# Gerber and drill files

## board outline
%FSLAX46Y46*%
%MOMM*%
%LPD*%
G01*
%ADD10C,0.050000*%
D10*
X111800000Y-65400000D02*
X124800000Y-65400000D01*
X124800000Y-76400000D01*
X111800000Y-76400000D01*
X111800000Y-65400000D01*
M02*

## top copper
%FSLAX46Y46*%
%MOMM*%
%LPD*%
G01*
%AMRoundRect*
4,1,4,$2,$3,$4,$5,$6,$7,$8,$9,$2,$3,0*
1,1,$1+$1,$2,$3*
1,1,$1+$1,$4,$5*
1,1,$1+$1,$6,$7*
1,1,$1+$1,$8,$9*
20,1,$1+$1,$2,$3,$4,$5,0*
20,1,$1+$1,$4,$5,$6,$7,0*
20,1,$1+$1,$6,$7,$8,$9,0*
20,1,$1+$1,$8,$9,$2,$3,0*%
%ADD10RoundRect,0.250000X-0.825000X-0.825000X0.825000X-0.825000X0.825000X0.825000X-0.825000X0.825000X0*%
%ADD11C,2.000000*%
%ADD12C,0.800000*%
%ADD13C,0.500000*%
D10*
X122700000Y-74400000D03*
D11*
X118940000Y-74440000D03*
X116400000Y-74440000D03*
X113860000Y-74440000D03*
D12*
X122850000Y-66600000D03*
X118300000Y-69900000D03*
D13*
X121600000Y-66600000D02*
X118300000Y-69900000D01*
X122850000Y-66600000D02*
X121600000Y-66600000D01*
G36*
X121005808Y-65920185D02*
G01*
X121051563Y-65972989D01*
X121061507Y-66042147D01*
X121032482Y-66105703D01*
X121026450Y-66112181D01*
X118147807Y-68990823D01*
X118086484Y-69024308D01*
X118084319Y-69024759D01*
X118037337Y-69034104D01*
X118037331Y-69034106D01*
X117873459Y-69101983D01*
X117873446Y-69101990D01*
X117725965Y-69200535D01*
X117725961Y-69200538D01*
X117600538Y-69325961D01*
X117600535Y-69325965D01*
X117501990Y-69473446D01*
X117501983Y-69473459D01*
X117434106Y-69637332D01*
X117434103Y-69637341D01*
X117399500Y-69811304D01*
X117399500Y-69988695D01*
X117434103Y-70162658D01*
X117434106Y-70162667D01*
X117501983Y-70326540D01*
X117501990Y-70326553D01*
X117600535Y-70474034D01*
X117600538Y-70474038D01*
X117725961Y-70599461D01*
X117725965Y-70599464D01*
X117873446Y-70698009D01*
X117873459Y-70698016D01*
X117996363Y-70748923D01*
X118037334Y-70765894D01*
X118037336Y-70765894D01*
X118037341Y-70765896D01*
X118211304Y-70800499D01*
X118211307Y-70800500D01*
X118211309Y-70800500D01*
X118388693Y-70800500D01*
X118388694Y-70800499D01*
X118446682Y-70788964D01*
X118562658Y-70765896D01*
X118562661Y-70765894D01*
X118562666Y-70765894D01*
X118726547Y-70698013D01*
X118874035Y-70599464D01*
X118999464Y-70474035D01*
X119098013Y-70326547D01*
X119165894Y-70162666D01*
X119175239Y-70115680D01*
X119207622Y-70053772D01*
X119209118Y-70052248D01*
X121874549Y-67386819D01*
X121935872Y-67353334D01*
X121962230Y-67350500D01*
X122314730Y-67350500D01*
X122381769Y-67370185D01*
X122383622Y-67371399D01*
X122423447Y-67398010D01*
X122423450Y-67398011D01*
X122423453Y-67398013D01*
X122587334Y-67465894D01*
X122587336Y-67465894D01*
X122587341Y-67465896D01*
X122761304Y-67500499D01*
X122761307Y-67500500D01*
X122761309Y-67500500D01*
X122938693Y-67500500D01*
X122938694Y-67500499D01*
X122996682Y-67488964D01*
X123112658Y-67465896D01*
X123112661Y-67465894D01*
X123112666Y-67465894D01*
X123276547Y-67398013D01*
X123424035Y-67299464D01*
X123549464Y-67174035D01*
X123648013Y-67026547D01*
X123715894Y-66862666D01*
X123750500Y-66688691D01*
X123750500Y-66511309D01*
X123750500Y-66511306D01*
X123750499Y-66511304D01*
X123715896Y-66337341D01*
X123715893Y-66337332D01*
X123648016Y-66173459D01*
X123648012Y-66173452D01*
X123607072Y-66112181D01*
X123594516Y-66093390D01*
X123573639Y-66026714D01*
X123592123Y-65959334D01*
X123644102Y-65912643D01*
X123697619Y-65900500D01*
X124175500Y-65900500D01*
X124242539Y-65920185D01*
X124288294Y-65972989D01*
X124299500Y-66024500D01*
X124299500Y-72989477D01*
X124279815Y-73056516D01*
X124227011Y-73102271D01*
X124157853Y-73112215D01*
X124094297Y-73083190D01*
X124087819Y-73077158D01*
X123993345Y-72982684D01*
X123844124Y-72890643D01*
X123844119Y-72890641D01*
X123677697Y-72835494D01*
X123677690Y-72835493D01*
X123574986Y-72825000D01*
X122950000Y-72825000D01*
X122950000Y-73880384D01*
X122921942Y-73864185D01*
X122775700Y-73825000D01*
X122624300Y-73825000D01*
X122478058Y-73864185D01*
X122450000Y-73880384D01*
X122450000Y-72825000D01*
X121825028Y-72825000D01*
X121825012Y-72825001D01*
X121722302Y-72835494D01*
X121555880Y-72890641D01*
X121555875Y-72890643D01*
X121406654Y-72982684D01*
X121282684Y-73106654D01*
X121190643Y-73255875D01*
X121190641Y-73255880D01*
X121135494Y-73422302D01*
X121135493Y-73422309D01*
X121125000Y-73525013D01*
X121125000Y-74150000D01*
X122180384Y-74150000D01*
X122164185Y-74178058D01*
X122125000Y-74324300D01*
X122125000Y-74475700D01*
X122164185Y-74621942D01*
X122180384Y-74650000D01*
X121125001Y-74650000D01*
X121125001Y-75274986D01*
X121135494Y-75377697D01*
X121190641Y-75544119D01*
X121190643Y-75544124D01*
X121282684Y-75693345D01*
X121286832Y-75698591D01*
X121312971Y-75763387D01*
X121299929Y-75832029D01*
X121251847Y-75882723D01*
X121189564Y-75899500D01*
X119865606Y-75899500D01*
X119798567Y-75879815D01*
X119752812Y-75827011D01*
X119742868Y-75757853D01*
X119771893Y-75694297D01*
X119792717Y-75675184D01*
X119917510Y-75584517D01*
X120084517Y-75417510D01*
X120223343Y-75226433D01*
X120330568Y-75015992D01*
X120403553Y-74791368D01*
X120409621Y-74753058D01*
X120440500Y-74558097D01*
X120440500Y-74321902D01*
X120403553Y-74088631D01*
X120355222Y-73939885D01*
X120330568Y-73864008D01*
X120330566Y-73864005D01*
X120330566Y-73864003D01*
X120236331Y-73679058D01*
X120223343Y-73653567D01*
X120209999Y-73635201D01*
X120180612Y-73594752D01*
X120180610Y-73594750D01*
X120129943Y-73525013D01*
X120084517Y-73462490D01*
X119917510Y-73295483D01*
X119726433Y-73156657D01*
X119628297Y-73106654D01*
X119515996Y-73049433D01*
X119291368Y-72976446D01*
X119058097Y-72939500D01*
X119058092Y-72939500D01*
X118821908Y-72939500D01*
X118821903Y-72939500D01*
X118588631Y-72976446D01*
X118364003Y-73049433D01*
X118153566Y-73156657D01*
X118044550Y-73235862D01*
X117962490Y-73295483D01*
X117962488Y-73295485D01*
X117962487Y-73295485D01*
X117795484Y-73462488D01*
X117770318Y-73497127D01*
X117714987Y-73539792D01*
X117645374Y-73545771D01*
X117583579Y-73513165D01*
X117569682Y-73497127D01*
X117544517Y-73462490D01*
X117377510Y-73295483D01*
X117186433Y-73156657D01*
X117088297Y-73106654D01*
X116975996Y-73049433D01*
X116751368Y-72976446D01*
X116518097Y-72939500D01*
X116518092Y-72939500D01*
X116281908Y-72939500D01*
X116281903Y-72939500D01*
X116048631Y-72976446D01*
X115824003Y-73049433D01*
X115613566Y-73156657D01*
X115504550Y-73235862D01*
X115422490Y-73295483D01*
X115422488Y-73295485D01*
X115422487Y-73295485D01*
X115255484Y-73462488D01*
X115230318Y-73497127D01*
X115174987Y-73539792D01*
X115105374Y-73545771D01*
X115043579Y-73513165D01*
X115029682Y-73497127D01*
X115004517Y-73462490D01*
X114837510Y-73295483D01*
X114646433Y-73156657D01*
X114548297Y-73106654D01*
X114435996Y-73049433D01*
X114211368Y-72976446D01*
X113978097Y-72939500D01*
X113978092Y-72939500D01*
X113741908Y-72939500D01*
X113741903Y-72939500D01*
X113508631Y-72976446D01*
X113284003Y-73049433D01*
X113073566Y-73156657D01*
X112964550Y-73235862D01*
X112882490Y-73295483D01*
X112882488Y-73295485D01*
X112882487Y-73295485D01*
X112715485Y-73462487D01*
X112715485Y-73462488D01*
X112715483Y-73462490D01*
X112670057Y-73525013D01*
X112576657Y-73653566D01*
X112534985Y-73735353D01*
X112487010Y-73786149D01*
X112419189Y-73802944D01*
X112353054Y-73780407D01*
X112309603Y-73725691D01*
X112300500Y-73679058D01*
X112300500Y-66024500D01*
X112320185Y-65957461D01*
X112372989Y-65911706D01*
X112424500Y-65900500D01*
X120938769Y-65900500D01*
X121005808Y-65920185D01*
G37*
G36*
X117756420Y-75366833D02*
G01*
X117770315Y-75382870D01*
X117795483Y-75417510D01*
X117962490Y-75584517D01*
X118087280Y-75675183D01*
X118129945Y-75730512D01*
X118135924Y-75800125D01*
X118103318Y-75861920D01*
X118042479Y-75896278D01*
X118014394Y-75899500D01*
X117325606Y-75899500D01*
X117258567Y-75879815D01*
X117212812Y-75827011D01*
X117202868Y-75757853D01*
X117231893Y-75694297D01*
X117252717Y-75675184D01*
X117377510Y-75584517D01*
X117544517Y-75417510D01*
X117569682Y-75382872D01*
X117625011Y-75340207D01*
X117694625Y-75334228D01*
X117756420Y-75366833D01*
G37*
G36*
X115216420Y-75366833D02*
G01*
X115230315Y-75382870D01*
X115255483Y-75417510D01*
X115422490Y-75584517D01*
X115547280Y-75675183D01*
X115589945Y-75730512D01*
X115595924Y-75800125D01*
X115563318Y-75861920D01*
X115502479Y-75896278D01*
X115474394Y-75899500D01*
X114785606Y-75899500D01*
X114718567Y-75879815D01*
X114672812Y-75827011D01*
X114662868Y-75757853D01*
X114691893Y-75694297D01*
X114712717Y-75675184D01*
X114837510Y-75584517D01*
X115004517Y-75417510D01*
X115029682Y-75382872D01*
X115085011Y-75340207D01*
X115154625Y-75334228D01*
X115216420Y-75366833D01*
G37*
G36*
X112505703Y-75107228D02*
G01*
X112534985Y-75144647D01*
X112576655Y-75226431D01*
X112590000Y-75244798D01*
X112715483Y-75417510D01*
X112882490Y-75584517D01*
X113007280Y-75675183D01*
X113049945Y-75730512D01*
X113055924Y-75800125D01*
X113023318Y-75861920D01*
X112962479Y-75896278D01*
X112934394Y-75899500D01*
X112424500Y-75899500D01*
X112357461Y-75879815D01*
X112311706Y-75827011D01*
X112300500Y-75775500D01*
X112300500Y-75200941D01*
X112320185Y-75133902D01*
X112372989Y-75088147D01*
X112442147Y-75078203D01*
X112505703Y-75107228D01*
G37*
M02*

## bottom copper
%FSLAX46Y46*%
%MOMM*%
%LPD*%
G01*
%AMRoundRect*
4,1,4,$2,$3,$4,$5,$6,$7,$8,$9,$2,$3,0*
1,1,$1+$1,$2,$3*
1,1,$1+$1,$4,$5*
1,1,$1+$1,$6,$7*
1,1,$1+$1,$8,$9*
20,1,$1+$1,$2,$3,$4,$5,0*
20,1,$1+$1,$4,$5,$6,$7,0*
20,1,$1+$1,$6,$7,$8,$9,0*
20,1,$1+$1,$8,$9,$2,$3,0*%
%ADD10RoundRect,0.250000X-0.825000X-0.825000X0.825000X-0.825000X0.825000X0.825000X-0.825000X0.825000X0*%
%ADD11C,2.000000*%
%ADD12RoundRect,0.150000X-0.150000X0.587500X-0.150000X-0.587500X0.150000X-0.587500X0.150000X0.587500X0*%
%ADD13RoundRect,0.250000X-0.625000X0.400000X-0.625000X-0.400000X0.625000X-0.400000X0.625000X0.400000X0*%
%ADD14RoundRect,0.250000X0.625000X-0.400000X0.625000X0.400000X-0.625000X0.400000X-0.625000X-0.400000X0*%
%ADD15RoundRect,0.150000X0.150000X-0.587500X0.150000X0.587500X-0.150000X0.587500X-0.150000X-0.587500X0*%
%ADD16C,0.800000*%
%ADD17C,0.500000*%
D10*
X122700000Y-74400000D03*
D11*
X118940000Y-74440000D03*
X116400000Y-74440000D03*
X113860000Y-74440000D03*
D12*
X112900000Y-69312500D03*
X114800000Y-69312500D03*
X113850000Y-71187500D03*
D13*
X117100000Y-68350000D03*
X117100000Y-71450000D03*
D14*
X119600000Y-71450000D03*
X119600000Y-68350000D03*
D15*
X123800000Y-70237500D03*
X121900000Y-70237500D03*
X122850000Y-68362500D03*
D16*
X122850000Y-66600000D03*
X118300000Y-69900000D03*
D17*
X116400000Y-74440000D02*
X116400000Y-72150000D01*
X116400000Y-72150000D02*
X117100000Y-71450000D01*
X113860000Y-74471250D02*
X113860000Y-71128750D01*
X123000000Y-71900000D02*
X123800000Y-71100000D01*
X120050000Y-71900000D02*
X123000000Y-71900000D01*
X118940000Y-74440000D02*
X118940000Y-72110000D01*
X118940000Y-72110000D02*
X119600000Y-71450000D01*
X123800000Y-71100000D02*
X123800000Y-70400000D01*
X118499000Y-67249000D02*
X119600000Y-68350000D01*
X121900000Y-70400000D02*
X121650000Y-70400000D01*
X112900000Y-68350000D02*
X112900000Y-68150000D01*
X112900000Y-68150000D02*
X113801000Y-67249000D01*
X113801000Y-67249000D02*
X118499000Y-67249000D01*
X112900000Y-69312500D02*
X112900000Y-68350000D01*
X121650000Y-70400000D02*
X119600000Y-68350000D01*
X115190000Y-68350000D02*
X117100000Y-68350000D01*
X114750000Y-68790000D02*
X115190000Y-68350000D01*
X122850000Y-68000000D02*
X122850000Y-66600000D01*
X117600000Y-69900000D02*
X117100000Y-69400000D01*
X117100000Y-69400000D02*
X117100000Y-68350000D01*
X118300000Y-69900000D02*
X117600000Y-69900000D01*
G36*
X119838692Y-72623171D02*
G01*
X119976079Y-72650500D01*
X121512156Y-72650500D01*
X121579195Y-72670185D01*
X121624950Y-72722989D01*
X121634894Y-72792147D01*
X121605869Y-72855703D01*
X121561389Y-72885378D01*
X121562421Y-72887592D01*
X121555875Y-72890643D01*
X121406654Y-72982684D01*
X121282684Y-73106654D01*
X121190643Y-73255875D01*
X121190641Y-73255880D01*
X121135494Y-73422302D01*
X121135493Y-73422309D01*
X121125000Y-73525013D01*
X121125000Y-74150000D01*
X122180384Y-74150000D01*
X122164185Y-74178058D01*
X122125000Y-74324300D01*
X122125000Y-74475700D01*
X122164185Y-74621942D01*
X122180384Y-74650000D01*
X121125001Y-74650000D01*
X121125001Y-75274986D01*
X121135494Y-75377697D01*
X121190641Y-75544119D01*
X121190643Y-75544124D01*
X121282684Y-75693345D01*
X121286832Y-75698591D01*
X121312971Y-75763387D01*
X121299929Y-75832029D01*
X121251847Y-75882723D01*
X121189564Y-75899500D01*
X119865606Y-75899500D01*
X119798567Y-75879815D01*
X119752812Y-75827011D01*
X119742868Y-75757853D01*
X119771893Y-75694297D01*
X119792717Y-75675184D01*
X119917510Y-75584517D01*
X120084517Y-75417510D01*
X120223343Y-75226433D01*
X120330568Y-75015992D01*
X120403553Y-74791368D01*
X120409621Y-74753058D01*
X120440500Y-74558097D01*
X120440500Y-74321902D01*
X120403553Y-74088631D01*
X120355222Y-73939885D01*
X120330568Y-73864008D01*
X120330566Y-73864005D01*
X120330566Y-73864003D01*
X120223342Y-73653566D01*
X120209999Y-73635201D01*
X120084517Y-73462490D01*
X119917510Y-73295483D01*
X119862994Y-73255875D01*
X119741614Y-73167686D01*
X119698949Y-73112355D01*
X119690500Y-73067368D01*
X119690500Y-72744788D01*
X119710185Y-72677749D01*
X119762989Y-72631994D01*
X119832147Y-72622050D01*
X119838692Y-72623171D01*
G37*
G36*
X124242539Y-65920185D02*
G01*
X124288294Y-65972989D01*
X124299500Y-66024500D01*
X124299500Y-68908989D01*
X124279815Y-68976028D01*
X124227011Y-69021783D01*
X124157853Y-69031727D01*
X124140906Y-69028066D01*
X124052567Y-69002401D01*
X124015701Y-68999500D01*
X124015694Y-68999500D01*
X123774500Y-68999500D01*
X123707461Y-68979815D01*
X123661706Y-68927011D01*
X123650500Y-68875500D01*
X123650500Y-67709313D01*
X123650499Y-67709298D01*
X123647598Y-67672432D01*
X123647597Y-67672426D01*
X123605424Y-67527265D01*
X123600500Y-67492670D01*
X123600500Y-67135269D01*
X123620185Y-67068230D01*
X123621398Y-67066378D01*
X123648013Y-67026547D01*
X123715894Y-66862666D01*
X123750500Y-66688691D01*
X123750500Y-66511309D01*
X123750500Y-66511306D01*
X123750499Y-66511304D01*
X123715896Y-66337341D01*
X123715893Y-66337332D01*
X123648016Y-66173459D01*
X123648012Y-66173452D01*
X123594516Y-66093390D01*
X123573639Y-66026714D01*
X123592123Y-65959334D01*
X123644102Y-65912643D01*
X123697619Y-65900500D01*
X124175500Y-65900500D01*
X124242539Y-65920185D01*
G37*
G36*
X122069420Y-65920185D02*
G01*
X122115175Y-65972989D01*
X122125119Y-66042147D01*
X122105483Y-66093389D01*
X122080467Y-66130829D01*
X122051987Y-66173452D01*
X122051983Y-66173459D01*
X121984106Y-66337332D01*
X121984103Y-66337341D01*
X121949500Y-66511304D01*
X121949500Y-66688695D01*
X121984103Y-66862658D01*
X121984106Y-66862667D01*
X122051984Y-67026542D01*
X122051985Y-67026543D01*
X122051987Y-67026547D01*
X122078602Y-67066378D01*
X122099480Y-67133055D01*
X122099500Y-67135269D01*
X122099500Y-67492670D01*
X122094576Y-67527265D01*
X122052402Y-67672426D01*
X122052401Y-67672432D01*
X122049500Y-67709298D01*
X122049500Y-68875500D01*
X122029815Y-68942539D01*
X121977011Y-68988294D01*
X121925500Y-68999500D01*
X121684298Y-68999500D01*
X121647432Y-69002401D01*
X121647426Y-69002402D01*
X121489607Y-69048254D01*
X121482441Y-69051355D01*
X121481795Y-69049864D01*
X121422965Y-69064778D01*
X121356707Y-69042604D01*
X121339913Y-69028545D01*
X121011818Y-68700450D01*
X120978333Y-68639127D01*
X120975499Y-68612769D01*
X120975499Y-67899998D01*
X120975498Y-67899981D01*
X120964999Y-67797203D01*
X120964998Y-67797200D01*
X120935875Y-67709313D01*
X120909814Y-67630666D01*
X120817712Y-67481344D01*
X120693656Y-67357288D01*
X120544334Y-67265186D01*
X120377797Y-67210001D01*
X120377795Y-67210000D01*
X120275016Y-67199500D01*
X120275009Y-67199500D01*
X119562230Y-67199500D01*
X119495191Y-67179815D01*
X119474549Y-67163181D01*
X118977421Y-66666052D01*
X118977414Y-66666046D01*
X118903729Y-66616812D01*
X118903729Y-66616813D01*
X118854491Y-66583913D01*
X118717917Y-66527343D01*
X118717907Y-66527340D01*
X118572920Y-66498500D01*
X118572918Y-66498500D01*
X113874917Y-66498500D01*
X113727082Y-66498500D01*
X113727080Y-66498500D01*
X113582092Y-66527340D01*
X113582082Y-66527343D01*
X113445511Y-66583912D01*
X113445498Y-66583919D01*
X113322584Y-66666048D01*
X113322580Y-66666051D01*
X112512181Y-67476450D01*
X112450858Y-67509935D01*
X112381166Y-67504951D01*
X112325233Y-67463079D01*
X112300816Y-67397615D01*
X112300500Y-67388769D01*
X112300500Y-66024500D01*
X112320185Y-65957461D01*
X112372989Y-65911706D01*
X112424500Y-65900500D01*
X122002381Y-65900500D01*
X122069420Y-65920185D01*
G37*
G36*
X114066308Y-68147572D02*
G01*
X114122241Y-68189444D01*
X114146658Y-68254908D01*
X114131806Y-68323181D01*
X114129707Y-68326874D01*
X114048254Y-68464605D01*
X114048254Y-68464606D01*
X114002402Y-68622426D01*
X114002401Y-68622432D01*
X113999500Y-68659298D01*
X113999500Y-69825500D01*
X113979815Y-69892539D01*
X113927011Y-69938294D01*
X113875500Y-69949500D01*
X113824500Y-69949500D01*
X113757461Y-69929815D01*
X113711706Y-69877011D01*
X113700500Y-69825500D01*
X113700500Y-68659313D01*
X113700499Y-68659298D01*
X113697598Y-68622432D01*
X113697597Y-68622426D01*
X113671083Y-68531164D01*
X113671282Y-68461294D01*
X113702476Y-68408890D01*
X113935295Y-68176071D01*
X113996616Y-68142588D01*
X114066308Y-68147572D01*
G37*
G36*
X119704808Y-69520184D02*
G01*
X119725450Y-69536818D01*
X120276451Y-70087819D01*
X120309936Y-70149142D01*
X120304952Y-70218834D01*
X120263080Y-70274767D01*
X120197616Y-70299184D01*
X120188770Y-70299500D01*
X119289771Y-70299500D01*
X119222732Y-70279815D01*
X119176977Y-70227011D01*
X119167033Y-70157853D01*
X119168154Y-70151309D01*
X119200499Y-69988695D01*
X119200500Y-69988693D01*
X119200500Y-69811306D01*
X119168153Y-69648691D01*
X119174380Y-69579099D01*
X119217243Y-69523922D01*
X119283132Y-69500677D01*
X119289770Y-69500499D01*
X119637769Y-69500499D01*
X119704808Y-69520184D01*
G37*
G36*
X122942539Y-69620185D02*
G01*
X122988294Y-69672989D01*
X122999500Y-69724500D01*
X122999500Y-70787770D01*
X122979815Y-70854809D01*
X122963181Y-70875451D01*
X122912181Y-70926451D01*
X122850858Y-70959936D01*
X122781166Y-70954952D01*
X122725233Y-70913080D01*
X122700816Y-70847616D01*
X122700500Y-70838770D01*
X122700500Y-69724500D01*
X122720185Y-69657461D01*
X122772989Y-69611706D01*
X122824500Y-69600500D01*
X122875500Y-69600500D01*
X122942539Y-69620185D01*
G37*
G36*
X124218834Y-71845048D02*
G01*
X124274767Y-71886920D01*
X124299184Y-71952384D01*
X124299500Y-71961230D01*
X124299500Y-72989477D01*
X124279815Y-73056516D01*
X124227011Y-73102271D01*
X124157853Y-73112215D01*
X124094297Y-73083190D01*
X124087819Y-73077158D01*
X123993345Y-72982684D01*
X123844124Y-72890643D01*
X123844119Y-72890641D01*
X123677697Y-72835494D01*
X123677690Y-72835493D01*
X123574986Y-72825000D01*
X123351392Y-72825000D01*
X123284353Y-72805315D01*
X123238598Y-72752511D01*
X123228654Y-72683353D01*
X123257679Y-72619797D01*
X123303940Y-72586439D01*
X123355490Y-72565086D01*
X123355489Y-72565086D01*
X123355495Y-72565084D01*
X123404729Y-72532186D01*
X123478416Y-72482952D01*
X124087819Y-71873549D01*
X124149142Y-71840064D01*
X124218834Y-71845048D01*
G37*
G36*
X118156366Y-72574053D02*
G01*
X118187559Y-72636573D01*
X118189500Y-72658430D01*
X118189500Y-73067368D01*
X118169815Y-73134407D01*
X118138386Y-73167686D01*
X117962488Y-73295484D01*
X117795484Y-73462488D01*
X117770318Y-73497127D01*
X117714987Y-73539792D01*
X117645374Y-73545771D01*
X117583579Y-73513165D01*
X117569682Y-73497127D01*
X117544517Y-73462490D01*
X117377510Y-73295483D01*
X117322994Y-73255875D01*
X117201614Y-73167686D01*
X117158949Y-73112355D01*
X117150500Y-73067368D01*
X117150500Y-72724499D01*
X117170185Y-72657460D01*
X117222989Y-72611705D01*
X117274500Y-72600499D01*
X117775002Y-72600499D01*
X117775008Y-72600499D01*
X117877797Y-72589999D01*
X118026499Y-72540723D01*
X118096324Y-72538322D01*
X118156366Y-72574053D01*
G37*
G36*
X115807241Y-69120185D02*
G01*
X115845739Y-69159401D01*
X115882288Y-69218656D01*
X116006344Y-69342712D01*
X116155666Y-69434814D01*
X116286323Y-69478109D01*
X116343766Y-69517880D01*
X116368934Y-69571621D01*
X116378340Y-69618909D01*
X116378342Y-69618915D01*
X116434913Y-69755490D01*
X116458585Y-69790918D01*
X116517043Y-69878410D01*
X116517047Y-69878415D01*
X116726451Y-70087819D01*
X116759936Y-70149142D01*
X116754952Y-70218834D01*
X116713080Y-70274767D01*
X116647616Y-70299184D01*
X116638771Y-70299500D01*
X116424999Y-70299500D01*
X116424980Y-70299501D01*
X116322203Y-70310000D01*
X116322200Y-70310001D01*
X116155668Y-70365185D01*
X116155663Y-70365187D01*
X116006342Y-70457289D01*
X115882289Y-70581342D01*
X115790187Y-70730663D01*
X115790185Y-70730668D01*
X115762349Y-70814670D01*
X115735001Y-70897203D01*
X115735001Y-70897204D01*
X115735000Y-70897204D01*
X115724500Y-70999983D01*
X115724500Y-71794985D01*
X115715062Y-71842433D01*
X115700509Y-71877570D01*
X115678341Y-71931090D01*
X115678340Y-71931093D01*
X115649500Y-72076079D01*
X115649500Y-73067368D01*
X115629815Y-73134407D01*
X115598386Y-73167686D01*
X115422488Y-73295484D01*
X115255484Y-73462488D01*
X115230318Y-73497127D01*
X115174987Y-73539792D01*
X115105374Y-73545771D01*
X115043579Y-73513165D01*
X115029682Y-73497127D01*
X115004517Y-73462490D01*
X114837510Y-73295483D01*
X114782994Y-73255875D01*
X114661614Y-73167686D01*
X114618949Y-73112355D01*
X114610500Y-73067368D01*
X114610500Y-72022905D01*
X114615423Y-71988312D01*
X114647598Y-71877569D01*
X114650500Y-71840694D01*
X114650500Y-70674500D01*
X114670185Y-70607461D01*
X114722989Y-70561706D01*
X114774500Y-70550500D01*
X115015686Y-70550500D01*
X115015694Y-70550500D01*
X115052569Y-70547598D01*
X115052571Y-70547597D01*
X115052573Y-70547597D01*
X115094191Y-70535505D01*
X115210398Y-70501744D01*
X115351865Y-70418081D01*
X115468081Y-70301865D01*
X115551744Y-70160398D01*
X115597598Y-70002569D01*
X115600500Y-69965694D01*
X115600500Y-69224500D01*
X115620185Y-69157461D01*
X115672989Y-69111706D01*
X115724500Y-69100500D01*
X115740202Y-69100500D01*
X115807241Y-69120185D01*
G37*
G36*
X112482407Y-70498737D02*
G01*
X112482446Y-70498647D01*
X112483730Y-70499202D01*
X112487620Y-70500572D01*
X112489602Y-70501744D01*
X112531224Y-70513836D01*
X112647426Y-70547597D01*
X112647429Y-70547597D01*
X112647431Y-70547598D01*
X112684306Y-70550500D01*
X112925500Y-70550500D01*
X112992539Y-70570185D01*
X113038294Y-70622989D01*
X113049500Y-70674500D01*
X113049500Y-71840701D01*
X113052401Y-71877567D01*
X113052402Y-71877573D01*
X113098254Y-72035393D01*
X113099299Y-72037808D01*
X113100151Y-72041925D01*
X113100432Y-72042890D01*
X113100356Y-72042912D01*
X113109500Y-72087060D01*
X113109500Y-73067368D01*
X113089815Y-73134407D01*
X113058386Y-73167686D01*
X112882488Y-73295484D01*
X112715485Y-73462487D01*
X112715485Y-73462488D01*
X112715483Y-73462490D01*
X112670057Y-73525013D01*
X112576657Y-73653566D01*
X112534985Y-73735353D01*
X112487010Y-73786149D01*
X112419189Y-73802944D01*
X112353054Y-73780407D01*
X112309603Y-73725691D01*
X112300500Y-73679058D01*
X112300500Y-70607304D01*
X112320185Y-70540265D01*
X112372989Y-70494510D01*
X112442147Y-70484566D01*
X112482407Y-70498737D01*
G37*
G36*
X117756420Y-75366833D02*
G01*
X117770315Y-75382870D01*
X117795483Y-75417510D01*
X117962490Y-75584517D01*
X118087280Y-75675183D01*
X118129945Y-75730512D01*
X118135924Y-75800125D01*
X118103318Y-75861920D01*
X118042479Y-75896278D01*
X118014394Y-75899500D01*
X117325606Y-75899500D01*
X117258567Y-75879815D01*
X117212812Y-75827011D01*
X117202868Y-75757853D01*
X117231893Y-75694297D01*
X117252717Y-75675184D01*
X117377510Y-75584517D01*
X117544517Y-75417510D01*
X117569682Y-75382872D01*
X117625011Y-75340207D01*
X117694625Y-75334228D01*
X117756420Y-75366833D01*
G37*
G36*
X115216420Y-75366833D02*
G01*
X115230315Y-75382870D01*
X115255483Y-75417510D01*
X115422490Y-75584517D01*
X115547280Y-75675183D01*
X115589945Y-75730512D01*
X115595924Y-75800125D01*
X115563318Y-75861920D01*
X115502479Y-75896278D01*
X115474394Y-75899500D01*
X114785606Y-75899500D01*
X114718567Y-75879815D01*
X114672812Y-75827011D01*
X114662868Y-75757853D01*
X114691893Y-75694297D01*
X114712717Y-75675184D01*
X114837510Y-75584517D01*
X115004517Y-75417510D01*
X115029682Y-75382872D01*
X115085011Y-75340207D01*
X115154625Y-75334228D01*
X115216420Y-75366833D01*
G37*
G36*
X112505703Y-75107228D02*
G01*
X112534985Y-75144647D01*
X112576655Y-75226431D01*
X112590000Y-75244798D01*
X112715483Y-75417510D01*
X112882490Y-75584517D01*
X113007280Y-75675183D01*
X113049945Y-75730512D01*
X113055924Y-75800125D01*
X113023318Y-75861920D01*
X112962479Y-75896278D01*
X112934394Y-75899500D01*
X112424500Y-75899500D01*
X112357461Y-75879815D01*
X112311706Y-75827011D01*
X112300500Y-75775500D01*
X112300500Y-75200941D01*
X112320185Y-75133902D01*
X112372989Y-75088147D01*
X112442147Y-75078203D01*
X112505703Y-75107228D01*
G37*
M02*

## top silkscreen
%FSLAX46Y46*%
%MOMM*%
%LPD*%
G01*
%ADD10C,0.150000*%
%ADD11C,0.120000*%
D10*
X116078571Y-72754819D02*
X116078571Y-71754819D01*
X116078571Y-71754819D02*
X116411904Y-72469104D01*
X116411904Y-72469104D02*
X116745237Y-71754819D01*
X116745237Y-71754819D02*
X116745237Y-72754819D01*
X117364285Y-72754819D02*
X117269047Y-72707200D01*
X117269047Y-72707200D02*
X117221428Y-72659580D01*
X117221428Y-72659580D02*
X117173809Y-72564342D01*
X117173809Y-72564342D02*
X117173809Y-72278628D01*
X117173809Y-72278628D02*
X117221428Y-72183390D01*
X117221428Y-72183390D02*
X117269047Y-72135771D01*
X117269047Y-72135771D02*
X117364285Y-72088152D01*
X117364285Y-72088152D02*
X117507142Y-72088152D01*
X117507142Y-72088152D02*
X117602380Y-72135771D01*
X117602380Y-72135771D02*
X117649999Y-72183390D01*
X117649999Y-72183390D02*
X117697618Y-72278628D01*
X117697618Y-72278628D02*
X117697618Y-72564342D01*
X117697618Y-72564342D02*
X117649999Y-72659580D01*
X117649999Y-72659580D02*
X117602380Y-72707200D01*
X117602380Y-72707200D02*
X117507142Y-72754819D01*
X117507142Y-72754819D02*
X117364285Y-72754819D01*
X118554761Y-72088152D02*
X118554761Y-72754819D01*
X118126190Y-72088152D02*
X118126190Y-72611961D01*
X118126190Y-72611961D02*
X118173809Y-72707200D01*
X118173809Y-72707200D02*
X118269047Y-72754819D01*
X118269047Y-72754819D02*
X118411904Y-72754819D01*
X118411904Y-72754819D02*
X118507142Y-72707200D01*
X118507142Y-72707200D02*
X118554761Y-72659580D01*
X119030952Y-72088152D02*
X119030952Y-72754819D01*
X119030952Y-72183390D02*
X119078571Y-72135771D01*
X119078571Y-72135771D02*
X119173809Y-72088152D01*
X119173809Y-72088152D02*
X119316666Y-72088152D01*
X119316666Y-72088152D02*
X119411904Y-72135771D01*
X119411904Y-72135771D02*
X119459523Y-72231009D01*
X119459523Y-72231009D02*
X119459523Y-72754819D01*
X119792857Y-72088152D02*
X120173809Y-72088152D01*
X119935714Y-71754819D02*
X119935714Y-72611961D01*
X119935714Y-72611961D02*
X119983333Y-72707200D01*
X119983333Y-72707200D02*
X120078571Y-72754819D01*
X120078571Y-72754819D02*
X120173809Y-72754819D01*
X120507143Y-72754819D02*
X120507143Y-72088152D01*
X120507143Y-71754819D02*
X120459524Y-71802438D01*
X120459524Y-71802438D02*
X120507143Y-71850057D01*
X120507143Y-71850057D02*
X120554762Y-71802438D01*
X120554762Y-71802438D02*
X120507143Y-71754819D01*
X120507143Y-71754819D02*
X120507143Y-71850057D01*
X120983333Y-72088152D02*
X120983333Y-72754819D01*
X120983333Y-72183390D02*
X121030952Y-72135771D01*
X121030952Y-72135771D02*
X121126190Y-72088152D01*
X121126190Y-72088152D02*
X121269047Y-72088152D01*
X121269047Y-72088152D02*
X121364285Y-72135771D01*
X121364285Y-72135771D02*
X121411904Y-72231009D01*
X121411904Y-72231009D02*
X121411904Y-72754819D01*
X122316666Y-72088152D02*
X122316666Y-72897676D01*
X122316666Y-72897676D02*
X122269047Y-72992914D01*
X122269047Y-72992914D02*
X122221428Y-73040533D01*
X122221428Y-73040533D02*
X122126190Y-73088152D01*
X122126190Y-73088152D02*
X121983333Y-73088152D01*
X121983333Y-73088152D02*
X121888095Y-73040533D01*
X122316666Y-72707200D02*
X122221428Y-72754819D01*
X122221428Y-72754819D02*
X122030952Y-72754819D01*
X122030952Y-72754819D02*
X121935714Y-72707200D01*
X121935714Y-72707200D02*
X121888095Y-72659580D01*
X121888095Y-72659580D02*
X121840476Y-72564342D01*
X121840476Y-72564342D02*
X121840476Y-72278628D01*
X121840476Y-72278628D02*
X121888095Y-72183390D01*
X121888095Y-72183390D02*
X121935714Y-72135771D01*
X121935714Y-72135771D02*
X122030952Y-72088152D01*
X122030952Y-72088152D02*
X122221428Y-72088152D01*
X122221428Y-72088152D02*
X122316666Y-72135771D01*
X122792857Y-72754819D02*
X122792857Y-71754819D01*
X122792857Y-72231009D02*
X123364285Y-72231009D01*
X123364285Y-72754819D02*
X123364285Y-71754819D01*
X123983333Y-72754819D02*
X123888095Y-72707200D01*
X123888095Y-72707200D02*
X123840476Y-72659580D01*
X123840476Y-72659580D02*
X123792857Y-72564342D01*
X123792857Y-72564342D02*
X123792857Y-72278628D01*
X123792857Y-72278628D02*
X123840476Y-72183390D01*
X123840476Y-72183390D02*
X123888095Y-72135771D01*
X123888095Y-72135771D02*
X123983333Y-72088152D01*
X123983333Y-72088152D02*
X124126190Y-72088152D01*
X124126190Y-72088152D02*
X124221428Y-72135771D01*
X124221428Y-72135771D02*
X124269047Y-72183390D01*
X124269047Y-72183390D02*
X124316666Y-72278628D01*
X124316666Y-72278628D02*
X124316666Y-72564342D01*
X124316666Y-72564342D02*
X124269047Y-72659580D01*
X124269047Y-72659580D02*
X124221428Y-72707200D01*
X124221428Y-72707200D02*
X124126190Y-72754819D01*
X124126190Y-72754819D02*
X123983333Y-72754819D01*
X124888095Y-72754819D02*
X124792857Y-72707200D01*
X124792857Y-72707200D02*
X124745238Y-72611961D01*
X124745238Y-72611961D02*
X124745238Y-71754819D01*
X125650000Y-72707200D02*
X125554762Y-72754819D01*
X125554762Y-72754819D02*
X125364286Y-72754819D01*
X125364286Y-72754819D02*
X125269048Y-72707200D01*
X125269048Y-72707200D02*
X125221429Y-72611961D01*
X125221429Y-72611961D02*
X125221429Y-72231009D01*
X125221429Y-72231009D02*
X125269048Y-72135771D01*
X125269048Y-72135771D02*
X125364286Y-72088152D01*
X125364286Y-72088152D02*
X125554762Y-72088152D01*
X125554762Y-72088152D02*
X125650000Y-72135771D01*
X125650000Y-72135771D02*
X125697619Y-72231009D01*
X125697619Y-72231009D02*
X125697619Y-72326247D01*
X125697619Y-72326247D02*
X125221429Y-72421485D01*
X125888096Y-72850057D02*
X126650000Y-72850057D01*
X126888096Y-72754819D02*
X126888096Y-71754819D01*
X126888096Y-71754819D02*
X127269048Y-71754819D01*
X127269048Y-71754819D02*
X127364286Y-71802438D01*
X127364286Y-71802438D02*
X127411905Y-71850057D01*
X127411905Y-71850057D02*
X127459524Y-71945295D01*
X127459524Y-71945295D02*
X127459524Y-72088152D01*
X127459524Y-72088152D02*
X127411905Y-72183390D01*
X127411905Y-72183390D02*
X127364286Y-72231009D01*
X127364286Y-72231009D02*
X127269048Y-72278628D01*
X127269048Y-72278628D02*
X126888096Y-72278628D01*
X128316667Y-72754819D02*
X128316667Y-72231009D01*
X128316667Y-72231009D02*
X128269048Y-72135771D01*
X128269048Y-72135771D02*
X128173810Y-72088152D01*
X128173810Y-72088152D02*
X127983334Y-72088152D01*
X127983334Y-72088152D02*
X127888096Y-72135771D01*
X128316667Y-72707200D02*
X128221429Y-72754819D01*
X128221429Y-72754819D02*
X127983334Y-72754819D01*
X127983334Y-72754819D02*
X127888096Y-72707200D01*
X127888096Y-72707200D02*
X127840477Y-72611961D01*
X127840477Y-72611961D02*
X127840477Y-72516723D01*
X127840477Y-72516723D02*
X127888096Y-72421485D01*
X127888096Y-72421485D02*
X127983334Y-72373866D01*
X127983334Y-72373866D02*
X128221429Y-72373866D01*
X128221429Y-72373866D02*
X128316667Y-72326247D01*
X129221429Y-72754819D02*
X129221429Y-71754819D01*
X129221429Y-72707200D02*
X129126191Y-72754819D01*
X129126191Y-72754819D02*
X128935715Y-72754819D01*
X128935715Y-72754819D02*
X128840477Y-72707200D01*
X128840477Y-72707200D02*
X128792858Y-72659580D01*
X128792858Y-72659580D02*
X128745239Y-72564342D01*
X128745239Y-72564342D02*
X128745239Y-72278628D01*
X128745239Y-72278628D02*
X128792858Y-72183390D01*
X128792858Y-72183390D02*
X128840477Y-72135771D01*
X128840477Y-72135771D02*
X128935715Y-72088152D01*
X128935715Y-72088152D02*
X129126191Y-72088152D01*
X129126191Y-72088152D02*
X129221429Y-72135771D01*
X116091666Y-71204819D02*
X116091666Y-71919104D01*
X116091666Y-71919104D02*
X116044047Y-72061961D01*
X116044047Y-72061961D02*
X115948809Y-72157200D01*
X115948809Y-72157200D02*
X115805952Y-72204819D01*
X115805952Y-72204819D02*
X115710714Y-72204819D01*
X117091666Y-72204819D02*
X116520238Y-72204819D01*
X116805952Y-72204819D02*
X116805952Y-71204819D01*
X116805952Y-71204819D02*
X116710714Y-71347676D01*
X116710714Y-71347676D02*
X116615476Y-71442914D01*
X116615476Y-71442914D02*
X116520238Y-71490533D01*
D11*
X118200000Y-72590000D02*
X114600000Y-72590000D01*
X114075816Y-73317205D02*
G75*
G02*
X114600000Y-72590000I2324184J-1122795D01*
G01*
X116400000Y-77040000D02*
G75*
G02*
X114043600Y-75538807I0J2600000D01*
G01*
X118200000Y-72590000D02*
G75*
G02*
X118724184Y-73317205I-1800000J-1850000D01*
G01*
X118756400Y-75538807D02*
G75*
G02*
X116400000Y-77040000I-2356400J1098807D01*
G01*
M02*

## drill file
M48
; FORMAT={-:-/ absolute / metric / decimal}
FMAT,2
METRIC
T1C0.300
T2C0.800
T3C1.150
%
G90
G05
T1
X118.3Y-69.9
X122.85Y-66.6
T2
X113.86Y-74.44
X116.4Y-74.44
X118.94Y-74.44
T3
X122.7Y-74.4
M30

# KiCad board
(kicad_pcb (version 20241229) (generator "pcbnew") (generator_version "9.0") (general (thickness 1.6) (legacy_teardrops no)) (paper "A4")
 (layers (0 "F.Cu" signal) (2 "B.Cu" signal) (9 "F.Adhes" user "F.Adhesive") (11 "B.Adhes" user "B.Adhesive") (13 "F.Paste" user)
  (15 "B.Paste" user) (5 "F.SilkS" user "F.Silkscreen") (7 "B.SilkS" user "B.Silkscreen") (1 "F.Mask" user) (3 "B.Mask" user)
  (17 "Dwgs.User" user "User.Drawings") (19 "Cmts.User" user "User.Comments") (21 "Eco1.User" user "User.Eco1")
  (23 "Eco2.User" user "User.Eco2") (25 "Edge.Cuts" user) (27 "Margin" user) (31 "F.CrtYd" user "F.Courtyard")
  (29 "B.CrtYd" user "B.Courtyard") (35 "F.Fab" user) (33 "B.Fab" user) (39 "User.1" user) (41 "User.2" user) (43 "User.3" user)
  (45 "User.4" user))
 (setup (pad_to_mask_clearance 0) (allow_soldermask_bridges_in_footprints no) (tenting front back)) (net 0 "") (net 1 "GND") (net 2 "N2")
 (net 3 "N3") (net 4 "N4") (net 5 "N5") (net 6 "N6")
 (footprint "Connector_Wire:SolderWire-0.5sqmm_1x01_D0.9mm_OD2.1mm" (layer "F.Cu") (at 122.7 74.4)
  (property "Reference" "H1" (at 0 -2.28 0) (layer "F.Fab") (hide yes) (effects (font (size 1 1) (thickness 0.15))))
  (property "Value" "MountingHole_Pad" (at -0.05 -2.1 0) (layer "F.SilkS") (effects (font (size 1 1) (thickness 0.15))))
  (pad "1" thru_hole roundrect (at 0 0) (size 2.15 2.15) (drill 1.15) (layers "*.Cu" "*.Mask") (remove_unused_layers no)
   (roundrect_rratio 0.116279) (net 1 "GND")))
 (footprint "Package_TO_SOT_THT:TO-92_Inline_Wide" (layer "F.Cu") (at 118.94 74.44 180)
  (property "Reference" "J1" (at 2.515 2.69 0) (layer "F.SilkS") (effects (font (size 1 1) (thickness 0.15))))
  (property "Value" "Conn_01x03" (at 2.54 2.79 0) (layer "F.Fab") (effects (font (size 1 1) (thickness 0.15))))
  (fp_line (start 0.74 1.85) (end 4.34 1.85) (stroke (width 0.12) (type solid)) (layer "F.SilkS"))
  (fp_arc (start 4.864184 1.122795) (mid 4.633903 1.509328) (end 4.34 1.85) (stroke (width 0.12) (type solid)) (layer "F.SilkS"))
  (fp_arc (start 2.54 -2.6) (mid 3.936979 -2.192818) (end 4.8964 -1.098807) (stroke (width 0.12) (type solid)) (layer "F.SilkS"))
  (fp_arc (start 0.74 1.85) (mid 0.446097 1.509328) (end 0.215816 1.122795) (stroke (width 0.12) (type solid)) (layer "F.SilkS"))
  (fp_arc (start 0.1836 -1.098807) (mid 1.143021 -2.192817) (end 2.54 -2.6) (stroke (width 0.12) (type solid)) (layer "F.SilkS"))
  (pad "1" thru_hole circle (at 0 0 180) (size 2 2) (drill 0.8) (layers "*.Cu" "*.Mask") (remove_unused_layers no) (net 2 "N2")
   (thermal_bridge_angle 90))
  (pad "2" thru_hole circle (at 2.54 0 180) (size 2 2) (drill 0.8) (layers "*.Cu" "*.Mask") (remove_unused_layers no) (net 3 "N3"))
  (pad "3" thru_hole circle (at 5.08 0 180) (size 2 2) (drill 0.8) (layers "*.Cu" "*.Mask") (remove_unused_layers no) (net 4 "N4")))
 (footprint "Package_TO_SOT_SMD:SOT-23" (layer "B.Cu") (at 113.85 70.25 -90)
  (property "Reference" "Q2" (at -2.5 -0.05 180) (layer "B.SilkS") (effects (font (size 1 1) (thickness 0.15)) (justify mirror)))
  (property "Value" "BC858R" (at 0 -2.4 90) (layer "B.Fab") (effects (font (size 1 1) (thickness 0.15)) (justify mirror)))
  (pad "1" smd roundrect (at -0.9375 0.95 270) (size 1.475 0.6) (layers "B.Cu" "B.Mask" "B.Paste") (roundrect_rratio 0.25) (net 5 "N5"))
  (pad "2" smd roundrect (at -0.9375 -0.95 270) (size 1.475 0.6) (layers "B.Cu" "B.Mask" "B.Paste") (roundrect_rratio 0.25) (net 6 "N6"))
  (pad "3" smd roundrect (at 0.9375 0 270) (size 1.475 0.6) (layers "B.Cu" "B.Mask" "B.Paste") (roundrect_rratio 0.25) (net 4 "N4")))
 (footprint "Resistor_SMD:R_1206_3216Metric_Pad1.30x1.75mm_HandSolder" (layer "B.Cu") (at 117.1 69.9 -90)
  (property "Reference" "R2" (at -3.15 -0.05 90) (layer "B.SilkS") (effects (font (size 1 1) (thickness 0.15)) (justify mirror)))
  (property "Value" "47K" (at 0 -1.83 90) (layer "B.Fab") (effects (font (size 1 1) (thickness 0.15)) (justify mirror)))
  (pad "1" smd roundrect (at -1.55 0 270) (size 1.3 1.75) (layers "B.Cu" "B.Mask" "B.Paste") (roundrect_rratio 0.192308) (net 6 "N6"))
  (pad "2" smd roundrect (at 1.55 0 270) (size 1.3 1.75) (layers "B.Cu" "B.Mask" "B.Paste") (roundrect_rratio 0.192308) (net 3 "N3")))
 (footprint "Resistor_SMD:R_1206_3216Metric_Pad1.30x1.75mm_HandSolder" (layer "B.Cu") (at 119.6 69.9 90)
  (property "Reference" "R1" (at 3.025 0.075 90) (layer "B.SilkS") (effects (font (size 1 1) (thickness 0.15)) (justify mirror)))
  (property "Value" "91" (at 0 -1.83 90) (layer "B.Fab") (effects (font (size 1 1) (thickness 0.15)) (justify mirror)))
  (pad "1" smd roundrect (at -1.55 0 90) (size 1.3 1.75) (layers "B.Cu" "B.Mask" "B.Paste") (roundrect_rratio 0.192308) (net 2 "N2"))
  (pad "2" smd roundrect (at 1.55 0 90) (size 1.3 1.75) (layers "B.Cu" "B.Mask" "B.Paste") (roundrect_rratio 0.192308) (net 5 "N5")))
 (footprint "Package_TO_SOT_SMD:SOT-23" (layer "B.Cu") (at 122.85 69.3 90)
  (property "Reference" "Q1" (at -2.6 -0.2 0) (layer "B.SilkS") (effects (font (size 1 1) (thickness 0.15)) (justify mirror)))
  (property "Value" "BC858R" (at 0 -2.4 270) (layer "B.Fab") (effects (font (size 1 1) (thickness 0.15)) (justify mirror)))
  (pad "1" smd roundrect (at -0.9375 0.95 90) (size 1.475 0.6) (layers "B.Cu" "B.Mask" "B.Paste") (roundrect_rratio 0.25) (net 2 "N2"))
  (pad "2" smd roundrect (at -0.9375 -0.95 90) (size 1.475 0.6) (layers "B.Cu" "B.Mask" "B.Paste") (roundrect_rratio 0.25) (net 5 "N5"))
  (pad "3" smd roundrect (at 0.9375 0 90) (size 1.475 0.6) (layers "B.Cu" "B.Mask" "B.Paste") (roundrect_rratio 0.25) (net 6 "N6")))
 (gr_rect (start 111.8 65.4) (end 124.8 76.4) (stroke (width 0.05) (type solid)) (fill no) (layer "Edge.Cuts"))
 (segment (start 116.4 74.44) (end 116.4 72.15) (width 0.5) (layer "B.Cu") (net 3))
 (segment (start 116.4 72.15) (end 117.1 71.45) (width 0.5) (layer "B.Cu") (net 3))
 (segment (start 113.86 74.47125) (end 113.86 71.12875) (width 0.5) (layer "B.Cu") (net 4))
 (segment (start 123 71.9) (end 123.8 71.1) (width 0.5) (layer "B.Cu") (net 2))
 (segment (start 120.05 71.9) (end 123 71.9) (width 0.5) (layer "B.Cu") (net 2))
 (segment (start 118.94 74.44) (end 118.94 72.11) (width 0.5) (layer "B.Cu") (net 2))
 (segment (start 118.94 72.11) (end 119.6 71.45) (width 0.5) (layer "B.Cu") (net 2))
 (segment (start 123.8 71.1) (end 123.8 70.4) (width 0.5) (layer "B.Cu") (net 2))
 (segment (start 118.499 67.249) (end 119.6 68.35) (width 0.5) (layer "B.Cu") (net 5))
 (segment (start 121.9 70.4) (end 121.65 70.4) (width 0.5) (layer "B.Cu") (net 5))
 (segment (start 112.9 68.35) (end 112.9 68.15) (width 0.5) (layer "B.Cu") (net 5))
 (segment (start 112.9 68.15) (end 113.801 67.249) (width 0.5) (layer "B.Cu") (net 5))
 (segment (start 113.801 67.249) (end 118.499 67.249) (width 0.5) (layer "B.Cu") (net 5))
 (segment (start 112.9 69.3125) (end 112.9 68.35) (width 0.5) (layer "B.Cu") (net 5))
 (segment (start 121.65 70.4) (end 119.6 68.35) (width 0.5) (layer "B.Cu") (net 5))
 (segment (start 121.6 66.6) (end 118.3 69.9) (width 0.5) (layer "F.Cu") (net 6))
 (segment (start 122.85 66.6) (end 121.6 66.6) (width 0.5) (layer "F.Cu") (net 6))
 (via (at 122.85 66.6) (size 0.8) (drill 0.3) (layers "F.Cu" "B.Cu") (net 6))
 (via (at 118.3 69.9) (size 0.8) (drill 0.3) (layers "F.Cu" "B.Cu") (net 6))
 (segment (start 115.19 68.35) (end 117.1 68.35) (width 0.5) (layer "B.Cu") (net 6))
 (segment (start 114.75 68.79) (end 115.19 68.35) (width 0.5) (layer "B.Cu") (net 6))
 (segment (start 122.85 68) (end 122.85 66.6) (width 0.5) (layer "B.Cu") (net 6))
 (segment (start 117.6 69.9) (end 117.1 69.4) (width 0.5) (layer "B.Cu") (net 6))
 (segment (start 117.1 69.4) (end 117.1 68.35) (width 0.5) (layer "B.Cu") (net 6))
 (segment (start 118.3 69.9) (end 117.6 69.9) (width 0.5) (layer "B.Cu") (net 6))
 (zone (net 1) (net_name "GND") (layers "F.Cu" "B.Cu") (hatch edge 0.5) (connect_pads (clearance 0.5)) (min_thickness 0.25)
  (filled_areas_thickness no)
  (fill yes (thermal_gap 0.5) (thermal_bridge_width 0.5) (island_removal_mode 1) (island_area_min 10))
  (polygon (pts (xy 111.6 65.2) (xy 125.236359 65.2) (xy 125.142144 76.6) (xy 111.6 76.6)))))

